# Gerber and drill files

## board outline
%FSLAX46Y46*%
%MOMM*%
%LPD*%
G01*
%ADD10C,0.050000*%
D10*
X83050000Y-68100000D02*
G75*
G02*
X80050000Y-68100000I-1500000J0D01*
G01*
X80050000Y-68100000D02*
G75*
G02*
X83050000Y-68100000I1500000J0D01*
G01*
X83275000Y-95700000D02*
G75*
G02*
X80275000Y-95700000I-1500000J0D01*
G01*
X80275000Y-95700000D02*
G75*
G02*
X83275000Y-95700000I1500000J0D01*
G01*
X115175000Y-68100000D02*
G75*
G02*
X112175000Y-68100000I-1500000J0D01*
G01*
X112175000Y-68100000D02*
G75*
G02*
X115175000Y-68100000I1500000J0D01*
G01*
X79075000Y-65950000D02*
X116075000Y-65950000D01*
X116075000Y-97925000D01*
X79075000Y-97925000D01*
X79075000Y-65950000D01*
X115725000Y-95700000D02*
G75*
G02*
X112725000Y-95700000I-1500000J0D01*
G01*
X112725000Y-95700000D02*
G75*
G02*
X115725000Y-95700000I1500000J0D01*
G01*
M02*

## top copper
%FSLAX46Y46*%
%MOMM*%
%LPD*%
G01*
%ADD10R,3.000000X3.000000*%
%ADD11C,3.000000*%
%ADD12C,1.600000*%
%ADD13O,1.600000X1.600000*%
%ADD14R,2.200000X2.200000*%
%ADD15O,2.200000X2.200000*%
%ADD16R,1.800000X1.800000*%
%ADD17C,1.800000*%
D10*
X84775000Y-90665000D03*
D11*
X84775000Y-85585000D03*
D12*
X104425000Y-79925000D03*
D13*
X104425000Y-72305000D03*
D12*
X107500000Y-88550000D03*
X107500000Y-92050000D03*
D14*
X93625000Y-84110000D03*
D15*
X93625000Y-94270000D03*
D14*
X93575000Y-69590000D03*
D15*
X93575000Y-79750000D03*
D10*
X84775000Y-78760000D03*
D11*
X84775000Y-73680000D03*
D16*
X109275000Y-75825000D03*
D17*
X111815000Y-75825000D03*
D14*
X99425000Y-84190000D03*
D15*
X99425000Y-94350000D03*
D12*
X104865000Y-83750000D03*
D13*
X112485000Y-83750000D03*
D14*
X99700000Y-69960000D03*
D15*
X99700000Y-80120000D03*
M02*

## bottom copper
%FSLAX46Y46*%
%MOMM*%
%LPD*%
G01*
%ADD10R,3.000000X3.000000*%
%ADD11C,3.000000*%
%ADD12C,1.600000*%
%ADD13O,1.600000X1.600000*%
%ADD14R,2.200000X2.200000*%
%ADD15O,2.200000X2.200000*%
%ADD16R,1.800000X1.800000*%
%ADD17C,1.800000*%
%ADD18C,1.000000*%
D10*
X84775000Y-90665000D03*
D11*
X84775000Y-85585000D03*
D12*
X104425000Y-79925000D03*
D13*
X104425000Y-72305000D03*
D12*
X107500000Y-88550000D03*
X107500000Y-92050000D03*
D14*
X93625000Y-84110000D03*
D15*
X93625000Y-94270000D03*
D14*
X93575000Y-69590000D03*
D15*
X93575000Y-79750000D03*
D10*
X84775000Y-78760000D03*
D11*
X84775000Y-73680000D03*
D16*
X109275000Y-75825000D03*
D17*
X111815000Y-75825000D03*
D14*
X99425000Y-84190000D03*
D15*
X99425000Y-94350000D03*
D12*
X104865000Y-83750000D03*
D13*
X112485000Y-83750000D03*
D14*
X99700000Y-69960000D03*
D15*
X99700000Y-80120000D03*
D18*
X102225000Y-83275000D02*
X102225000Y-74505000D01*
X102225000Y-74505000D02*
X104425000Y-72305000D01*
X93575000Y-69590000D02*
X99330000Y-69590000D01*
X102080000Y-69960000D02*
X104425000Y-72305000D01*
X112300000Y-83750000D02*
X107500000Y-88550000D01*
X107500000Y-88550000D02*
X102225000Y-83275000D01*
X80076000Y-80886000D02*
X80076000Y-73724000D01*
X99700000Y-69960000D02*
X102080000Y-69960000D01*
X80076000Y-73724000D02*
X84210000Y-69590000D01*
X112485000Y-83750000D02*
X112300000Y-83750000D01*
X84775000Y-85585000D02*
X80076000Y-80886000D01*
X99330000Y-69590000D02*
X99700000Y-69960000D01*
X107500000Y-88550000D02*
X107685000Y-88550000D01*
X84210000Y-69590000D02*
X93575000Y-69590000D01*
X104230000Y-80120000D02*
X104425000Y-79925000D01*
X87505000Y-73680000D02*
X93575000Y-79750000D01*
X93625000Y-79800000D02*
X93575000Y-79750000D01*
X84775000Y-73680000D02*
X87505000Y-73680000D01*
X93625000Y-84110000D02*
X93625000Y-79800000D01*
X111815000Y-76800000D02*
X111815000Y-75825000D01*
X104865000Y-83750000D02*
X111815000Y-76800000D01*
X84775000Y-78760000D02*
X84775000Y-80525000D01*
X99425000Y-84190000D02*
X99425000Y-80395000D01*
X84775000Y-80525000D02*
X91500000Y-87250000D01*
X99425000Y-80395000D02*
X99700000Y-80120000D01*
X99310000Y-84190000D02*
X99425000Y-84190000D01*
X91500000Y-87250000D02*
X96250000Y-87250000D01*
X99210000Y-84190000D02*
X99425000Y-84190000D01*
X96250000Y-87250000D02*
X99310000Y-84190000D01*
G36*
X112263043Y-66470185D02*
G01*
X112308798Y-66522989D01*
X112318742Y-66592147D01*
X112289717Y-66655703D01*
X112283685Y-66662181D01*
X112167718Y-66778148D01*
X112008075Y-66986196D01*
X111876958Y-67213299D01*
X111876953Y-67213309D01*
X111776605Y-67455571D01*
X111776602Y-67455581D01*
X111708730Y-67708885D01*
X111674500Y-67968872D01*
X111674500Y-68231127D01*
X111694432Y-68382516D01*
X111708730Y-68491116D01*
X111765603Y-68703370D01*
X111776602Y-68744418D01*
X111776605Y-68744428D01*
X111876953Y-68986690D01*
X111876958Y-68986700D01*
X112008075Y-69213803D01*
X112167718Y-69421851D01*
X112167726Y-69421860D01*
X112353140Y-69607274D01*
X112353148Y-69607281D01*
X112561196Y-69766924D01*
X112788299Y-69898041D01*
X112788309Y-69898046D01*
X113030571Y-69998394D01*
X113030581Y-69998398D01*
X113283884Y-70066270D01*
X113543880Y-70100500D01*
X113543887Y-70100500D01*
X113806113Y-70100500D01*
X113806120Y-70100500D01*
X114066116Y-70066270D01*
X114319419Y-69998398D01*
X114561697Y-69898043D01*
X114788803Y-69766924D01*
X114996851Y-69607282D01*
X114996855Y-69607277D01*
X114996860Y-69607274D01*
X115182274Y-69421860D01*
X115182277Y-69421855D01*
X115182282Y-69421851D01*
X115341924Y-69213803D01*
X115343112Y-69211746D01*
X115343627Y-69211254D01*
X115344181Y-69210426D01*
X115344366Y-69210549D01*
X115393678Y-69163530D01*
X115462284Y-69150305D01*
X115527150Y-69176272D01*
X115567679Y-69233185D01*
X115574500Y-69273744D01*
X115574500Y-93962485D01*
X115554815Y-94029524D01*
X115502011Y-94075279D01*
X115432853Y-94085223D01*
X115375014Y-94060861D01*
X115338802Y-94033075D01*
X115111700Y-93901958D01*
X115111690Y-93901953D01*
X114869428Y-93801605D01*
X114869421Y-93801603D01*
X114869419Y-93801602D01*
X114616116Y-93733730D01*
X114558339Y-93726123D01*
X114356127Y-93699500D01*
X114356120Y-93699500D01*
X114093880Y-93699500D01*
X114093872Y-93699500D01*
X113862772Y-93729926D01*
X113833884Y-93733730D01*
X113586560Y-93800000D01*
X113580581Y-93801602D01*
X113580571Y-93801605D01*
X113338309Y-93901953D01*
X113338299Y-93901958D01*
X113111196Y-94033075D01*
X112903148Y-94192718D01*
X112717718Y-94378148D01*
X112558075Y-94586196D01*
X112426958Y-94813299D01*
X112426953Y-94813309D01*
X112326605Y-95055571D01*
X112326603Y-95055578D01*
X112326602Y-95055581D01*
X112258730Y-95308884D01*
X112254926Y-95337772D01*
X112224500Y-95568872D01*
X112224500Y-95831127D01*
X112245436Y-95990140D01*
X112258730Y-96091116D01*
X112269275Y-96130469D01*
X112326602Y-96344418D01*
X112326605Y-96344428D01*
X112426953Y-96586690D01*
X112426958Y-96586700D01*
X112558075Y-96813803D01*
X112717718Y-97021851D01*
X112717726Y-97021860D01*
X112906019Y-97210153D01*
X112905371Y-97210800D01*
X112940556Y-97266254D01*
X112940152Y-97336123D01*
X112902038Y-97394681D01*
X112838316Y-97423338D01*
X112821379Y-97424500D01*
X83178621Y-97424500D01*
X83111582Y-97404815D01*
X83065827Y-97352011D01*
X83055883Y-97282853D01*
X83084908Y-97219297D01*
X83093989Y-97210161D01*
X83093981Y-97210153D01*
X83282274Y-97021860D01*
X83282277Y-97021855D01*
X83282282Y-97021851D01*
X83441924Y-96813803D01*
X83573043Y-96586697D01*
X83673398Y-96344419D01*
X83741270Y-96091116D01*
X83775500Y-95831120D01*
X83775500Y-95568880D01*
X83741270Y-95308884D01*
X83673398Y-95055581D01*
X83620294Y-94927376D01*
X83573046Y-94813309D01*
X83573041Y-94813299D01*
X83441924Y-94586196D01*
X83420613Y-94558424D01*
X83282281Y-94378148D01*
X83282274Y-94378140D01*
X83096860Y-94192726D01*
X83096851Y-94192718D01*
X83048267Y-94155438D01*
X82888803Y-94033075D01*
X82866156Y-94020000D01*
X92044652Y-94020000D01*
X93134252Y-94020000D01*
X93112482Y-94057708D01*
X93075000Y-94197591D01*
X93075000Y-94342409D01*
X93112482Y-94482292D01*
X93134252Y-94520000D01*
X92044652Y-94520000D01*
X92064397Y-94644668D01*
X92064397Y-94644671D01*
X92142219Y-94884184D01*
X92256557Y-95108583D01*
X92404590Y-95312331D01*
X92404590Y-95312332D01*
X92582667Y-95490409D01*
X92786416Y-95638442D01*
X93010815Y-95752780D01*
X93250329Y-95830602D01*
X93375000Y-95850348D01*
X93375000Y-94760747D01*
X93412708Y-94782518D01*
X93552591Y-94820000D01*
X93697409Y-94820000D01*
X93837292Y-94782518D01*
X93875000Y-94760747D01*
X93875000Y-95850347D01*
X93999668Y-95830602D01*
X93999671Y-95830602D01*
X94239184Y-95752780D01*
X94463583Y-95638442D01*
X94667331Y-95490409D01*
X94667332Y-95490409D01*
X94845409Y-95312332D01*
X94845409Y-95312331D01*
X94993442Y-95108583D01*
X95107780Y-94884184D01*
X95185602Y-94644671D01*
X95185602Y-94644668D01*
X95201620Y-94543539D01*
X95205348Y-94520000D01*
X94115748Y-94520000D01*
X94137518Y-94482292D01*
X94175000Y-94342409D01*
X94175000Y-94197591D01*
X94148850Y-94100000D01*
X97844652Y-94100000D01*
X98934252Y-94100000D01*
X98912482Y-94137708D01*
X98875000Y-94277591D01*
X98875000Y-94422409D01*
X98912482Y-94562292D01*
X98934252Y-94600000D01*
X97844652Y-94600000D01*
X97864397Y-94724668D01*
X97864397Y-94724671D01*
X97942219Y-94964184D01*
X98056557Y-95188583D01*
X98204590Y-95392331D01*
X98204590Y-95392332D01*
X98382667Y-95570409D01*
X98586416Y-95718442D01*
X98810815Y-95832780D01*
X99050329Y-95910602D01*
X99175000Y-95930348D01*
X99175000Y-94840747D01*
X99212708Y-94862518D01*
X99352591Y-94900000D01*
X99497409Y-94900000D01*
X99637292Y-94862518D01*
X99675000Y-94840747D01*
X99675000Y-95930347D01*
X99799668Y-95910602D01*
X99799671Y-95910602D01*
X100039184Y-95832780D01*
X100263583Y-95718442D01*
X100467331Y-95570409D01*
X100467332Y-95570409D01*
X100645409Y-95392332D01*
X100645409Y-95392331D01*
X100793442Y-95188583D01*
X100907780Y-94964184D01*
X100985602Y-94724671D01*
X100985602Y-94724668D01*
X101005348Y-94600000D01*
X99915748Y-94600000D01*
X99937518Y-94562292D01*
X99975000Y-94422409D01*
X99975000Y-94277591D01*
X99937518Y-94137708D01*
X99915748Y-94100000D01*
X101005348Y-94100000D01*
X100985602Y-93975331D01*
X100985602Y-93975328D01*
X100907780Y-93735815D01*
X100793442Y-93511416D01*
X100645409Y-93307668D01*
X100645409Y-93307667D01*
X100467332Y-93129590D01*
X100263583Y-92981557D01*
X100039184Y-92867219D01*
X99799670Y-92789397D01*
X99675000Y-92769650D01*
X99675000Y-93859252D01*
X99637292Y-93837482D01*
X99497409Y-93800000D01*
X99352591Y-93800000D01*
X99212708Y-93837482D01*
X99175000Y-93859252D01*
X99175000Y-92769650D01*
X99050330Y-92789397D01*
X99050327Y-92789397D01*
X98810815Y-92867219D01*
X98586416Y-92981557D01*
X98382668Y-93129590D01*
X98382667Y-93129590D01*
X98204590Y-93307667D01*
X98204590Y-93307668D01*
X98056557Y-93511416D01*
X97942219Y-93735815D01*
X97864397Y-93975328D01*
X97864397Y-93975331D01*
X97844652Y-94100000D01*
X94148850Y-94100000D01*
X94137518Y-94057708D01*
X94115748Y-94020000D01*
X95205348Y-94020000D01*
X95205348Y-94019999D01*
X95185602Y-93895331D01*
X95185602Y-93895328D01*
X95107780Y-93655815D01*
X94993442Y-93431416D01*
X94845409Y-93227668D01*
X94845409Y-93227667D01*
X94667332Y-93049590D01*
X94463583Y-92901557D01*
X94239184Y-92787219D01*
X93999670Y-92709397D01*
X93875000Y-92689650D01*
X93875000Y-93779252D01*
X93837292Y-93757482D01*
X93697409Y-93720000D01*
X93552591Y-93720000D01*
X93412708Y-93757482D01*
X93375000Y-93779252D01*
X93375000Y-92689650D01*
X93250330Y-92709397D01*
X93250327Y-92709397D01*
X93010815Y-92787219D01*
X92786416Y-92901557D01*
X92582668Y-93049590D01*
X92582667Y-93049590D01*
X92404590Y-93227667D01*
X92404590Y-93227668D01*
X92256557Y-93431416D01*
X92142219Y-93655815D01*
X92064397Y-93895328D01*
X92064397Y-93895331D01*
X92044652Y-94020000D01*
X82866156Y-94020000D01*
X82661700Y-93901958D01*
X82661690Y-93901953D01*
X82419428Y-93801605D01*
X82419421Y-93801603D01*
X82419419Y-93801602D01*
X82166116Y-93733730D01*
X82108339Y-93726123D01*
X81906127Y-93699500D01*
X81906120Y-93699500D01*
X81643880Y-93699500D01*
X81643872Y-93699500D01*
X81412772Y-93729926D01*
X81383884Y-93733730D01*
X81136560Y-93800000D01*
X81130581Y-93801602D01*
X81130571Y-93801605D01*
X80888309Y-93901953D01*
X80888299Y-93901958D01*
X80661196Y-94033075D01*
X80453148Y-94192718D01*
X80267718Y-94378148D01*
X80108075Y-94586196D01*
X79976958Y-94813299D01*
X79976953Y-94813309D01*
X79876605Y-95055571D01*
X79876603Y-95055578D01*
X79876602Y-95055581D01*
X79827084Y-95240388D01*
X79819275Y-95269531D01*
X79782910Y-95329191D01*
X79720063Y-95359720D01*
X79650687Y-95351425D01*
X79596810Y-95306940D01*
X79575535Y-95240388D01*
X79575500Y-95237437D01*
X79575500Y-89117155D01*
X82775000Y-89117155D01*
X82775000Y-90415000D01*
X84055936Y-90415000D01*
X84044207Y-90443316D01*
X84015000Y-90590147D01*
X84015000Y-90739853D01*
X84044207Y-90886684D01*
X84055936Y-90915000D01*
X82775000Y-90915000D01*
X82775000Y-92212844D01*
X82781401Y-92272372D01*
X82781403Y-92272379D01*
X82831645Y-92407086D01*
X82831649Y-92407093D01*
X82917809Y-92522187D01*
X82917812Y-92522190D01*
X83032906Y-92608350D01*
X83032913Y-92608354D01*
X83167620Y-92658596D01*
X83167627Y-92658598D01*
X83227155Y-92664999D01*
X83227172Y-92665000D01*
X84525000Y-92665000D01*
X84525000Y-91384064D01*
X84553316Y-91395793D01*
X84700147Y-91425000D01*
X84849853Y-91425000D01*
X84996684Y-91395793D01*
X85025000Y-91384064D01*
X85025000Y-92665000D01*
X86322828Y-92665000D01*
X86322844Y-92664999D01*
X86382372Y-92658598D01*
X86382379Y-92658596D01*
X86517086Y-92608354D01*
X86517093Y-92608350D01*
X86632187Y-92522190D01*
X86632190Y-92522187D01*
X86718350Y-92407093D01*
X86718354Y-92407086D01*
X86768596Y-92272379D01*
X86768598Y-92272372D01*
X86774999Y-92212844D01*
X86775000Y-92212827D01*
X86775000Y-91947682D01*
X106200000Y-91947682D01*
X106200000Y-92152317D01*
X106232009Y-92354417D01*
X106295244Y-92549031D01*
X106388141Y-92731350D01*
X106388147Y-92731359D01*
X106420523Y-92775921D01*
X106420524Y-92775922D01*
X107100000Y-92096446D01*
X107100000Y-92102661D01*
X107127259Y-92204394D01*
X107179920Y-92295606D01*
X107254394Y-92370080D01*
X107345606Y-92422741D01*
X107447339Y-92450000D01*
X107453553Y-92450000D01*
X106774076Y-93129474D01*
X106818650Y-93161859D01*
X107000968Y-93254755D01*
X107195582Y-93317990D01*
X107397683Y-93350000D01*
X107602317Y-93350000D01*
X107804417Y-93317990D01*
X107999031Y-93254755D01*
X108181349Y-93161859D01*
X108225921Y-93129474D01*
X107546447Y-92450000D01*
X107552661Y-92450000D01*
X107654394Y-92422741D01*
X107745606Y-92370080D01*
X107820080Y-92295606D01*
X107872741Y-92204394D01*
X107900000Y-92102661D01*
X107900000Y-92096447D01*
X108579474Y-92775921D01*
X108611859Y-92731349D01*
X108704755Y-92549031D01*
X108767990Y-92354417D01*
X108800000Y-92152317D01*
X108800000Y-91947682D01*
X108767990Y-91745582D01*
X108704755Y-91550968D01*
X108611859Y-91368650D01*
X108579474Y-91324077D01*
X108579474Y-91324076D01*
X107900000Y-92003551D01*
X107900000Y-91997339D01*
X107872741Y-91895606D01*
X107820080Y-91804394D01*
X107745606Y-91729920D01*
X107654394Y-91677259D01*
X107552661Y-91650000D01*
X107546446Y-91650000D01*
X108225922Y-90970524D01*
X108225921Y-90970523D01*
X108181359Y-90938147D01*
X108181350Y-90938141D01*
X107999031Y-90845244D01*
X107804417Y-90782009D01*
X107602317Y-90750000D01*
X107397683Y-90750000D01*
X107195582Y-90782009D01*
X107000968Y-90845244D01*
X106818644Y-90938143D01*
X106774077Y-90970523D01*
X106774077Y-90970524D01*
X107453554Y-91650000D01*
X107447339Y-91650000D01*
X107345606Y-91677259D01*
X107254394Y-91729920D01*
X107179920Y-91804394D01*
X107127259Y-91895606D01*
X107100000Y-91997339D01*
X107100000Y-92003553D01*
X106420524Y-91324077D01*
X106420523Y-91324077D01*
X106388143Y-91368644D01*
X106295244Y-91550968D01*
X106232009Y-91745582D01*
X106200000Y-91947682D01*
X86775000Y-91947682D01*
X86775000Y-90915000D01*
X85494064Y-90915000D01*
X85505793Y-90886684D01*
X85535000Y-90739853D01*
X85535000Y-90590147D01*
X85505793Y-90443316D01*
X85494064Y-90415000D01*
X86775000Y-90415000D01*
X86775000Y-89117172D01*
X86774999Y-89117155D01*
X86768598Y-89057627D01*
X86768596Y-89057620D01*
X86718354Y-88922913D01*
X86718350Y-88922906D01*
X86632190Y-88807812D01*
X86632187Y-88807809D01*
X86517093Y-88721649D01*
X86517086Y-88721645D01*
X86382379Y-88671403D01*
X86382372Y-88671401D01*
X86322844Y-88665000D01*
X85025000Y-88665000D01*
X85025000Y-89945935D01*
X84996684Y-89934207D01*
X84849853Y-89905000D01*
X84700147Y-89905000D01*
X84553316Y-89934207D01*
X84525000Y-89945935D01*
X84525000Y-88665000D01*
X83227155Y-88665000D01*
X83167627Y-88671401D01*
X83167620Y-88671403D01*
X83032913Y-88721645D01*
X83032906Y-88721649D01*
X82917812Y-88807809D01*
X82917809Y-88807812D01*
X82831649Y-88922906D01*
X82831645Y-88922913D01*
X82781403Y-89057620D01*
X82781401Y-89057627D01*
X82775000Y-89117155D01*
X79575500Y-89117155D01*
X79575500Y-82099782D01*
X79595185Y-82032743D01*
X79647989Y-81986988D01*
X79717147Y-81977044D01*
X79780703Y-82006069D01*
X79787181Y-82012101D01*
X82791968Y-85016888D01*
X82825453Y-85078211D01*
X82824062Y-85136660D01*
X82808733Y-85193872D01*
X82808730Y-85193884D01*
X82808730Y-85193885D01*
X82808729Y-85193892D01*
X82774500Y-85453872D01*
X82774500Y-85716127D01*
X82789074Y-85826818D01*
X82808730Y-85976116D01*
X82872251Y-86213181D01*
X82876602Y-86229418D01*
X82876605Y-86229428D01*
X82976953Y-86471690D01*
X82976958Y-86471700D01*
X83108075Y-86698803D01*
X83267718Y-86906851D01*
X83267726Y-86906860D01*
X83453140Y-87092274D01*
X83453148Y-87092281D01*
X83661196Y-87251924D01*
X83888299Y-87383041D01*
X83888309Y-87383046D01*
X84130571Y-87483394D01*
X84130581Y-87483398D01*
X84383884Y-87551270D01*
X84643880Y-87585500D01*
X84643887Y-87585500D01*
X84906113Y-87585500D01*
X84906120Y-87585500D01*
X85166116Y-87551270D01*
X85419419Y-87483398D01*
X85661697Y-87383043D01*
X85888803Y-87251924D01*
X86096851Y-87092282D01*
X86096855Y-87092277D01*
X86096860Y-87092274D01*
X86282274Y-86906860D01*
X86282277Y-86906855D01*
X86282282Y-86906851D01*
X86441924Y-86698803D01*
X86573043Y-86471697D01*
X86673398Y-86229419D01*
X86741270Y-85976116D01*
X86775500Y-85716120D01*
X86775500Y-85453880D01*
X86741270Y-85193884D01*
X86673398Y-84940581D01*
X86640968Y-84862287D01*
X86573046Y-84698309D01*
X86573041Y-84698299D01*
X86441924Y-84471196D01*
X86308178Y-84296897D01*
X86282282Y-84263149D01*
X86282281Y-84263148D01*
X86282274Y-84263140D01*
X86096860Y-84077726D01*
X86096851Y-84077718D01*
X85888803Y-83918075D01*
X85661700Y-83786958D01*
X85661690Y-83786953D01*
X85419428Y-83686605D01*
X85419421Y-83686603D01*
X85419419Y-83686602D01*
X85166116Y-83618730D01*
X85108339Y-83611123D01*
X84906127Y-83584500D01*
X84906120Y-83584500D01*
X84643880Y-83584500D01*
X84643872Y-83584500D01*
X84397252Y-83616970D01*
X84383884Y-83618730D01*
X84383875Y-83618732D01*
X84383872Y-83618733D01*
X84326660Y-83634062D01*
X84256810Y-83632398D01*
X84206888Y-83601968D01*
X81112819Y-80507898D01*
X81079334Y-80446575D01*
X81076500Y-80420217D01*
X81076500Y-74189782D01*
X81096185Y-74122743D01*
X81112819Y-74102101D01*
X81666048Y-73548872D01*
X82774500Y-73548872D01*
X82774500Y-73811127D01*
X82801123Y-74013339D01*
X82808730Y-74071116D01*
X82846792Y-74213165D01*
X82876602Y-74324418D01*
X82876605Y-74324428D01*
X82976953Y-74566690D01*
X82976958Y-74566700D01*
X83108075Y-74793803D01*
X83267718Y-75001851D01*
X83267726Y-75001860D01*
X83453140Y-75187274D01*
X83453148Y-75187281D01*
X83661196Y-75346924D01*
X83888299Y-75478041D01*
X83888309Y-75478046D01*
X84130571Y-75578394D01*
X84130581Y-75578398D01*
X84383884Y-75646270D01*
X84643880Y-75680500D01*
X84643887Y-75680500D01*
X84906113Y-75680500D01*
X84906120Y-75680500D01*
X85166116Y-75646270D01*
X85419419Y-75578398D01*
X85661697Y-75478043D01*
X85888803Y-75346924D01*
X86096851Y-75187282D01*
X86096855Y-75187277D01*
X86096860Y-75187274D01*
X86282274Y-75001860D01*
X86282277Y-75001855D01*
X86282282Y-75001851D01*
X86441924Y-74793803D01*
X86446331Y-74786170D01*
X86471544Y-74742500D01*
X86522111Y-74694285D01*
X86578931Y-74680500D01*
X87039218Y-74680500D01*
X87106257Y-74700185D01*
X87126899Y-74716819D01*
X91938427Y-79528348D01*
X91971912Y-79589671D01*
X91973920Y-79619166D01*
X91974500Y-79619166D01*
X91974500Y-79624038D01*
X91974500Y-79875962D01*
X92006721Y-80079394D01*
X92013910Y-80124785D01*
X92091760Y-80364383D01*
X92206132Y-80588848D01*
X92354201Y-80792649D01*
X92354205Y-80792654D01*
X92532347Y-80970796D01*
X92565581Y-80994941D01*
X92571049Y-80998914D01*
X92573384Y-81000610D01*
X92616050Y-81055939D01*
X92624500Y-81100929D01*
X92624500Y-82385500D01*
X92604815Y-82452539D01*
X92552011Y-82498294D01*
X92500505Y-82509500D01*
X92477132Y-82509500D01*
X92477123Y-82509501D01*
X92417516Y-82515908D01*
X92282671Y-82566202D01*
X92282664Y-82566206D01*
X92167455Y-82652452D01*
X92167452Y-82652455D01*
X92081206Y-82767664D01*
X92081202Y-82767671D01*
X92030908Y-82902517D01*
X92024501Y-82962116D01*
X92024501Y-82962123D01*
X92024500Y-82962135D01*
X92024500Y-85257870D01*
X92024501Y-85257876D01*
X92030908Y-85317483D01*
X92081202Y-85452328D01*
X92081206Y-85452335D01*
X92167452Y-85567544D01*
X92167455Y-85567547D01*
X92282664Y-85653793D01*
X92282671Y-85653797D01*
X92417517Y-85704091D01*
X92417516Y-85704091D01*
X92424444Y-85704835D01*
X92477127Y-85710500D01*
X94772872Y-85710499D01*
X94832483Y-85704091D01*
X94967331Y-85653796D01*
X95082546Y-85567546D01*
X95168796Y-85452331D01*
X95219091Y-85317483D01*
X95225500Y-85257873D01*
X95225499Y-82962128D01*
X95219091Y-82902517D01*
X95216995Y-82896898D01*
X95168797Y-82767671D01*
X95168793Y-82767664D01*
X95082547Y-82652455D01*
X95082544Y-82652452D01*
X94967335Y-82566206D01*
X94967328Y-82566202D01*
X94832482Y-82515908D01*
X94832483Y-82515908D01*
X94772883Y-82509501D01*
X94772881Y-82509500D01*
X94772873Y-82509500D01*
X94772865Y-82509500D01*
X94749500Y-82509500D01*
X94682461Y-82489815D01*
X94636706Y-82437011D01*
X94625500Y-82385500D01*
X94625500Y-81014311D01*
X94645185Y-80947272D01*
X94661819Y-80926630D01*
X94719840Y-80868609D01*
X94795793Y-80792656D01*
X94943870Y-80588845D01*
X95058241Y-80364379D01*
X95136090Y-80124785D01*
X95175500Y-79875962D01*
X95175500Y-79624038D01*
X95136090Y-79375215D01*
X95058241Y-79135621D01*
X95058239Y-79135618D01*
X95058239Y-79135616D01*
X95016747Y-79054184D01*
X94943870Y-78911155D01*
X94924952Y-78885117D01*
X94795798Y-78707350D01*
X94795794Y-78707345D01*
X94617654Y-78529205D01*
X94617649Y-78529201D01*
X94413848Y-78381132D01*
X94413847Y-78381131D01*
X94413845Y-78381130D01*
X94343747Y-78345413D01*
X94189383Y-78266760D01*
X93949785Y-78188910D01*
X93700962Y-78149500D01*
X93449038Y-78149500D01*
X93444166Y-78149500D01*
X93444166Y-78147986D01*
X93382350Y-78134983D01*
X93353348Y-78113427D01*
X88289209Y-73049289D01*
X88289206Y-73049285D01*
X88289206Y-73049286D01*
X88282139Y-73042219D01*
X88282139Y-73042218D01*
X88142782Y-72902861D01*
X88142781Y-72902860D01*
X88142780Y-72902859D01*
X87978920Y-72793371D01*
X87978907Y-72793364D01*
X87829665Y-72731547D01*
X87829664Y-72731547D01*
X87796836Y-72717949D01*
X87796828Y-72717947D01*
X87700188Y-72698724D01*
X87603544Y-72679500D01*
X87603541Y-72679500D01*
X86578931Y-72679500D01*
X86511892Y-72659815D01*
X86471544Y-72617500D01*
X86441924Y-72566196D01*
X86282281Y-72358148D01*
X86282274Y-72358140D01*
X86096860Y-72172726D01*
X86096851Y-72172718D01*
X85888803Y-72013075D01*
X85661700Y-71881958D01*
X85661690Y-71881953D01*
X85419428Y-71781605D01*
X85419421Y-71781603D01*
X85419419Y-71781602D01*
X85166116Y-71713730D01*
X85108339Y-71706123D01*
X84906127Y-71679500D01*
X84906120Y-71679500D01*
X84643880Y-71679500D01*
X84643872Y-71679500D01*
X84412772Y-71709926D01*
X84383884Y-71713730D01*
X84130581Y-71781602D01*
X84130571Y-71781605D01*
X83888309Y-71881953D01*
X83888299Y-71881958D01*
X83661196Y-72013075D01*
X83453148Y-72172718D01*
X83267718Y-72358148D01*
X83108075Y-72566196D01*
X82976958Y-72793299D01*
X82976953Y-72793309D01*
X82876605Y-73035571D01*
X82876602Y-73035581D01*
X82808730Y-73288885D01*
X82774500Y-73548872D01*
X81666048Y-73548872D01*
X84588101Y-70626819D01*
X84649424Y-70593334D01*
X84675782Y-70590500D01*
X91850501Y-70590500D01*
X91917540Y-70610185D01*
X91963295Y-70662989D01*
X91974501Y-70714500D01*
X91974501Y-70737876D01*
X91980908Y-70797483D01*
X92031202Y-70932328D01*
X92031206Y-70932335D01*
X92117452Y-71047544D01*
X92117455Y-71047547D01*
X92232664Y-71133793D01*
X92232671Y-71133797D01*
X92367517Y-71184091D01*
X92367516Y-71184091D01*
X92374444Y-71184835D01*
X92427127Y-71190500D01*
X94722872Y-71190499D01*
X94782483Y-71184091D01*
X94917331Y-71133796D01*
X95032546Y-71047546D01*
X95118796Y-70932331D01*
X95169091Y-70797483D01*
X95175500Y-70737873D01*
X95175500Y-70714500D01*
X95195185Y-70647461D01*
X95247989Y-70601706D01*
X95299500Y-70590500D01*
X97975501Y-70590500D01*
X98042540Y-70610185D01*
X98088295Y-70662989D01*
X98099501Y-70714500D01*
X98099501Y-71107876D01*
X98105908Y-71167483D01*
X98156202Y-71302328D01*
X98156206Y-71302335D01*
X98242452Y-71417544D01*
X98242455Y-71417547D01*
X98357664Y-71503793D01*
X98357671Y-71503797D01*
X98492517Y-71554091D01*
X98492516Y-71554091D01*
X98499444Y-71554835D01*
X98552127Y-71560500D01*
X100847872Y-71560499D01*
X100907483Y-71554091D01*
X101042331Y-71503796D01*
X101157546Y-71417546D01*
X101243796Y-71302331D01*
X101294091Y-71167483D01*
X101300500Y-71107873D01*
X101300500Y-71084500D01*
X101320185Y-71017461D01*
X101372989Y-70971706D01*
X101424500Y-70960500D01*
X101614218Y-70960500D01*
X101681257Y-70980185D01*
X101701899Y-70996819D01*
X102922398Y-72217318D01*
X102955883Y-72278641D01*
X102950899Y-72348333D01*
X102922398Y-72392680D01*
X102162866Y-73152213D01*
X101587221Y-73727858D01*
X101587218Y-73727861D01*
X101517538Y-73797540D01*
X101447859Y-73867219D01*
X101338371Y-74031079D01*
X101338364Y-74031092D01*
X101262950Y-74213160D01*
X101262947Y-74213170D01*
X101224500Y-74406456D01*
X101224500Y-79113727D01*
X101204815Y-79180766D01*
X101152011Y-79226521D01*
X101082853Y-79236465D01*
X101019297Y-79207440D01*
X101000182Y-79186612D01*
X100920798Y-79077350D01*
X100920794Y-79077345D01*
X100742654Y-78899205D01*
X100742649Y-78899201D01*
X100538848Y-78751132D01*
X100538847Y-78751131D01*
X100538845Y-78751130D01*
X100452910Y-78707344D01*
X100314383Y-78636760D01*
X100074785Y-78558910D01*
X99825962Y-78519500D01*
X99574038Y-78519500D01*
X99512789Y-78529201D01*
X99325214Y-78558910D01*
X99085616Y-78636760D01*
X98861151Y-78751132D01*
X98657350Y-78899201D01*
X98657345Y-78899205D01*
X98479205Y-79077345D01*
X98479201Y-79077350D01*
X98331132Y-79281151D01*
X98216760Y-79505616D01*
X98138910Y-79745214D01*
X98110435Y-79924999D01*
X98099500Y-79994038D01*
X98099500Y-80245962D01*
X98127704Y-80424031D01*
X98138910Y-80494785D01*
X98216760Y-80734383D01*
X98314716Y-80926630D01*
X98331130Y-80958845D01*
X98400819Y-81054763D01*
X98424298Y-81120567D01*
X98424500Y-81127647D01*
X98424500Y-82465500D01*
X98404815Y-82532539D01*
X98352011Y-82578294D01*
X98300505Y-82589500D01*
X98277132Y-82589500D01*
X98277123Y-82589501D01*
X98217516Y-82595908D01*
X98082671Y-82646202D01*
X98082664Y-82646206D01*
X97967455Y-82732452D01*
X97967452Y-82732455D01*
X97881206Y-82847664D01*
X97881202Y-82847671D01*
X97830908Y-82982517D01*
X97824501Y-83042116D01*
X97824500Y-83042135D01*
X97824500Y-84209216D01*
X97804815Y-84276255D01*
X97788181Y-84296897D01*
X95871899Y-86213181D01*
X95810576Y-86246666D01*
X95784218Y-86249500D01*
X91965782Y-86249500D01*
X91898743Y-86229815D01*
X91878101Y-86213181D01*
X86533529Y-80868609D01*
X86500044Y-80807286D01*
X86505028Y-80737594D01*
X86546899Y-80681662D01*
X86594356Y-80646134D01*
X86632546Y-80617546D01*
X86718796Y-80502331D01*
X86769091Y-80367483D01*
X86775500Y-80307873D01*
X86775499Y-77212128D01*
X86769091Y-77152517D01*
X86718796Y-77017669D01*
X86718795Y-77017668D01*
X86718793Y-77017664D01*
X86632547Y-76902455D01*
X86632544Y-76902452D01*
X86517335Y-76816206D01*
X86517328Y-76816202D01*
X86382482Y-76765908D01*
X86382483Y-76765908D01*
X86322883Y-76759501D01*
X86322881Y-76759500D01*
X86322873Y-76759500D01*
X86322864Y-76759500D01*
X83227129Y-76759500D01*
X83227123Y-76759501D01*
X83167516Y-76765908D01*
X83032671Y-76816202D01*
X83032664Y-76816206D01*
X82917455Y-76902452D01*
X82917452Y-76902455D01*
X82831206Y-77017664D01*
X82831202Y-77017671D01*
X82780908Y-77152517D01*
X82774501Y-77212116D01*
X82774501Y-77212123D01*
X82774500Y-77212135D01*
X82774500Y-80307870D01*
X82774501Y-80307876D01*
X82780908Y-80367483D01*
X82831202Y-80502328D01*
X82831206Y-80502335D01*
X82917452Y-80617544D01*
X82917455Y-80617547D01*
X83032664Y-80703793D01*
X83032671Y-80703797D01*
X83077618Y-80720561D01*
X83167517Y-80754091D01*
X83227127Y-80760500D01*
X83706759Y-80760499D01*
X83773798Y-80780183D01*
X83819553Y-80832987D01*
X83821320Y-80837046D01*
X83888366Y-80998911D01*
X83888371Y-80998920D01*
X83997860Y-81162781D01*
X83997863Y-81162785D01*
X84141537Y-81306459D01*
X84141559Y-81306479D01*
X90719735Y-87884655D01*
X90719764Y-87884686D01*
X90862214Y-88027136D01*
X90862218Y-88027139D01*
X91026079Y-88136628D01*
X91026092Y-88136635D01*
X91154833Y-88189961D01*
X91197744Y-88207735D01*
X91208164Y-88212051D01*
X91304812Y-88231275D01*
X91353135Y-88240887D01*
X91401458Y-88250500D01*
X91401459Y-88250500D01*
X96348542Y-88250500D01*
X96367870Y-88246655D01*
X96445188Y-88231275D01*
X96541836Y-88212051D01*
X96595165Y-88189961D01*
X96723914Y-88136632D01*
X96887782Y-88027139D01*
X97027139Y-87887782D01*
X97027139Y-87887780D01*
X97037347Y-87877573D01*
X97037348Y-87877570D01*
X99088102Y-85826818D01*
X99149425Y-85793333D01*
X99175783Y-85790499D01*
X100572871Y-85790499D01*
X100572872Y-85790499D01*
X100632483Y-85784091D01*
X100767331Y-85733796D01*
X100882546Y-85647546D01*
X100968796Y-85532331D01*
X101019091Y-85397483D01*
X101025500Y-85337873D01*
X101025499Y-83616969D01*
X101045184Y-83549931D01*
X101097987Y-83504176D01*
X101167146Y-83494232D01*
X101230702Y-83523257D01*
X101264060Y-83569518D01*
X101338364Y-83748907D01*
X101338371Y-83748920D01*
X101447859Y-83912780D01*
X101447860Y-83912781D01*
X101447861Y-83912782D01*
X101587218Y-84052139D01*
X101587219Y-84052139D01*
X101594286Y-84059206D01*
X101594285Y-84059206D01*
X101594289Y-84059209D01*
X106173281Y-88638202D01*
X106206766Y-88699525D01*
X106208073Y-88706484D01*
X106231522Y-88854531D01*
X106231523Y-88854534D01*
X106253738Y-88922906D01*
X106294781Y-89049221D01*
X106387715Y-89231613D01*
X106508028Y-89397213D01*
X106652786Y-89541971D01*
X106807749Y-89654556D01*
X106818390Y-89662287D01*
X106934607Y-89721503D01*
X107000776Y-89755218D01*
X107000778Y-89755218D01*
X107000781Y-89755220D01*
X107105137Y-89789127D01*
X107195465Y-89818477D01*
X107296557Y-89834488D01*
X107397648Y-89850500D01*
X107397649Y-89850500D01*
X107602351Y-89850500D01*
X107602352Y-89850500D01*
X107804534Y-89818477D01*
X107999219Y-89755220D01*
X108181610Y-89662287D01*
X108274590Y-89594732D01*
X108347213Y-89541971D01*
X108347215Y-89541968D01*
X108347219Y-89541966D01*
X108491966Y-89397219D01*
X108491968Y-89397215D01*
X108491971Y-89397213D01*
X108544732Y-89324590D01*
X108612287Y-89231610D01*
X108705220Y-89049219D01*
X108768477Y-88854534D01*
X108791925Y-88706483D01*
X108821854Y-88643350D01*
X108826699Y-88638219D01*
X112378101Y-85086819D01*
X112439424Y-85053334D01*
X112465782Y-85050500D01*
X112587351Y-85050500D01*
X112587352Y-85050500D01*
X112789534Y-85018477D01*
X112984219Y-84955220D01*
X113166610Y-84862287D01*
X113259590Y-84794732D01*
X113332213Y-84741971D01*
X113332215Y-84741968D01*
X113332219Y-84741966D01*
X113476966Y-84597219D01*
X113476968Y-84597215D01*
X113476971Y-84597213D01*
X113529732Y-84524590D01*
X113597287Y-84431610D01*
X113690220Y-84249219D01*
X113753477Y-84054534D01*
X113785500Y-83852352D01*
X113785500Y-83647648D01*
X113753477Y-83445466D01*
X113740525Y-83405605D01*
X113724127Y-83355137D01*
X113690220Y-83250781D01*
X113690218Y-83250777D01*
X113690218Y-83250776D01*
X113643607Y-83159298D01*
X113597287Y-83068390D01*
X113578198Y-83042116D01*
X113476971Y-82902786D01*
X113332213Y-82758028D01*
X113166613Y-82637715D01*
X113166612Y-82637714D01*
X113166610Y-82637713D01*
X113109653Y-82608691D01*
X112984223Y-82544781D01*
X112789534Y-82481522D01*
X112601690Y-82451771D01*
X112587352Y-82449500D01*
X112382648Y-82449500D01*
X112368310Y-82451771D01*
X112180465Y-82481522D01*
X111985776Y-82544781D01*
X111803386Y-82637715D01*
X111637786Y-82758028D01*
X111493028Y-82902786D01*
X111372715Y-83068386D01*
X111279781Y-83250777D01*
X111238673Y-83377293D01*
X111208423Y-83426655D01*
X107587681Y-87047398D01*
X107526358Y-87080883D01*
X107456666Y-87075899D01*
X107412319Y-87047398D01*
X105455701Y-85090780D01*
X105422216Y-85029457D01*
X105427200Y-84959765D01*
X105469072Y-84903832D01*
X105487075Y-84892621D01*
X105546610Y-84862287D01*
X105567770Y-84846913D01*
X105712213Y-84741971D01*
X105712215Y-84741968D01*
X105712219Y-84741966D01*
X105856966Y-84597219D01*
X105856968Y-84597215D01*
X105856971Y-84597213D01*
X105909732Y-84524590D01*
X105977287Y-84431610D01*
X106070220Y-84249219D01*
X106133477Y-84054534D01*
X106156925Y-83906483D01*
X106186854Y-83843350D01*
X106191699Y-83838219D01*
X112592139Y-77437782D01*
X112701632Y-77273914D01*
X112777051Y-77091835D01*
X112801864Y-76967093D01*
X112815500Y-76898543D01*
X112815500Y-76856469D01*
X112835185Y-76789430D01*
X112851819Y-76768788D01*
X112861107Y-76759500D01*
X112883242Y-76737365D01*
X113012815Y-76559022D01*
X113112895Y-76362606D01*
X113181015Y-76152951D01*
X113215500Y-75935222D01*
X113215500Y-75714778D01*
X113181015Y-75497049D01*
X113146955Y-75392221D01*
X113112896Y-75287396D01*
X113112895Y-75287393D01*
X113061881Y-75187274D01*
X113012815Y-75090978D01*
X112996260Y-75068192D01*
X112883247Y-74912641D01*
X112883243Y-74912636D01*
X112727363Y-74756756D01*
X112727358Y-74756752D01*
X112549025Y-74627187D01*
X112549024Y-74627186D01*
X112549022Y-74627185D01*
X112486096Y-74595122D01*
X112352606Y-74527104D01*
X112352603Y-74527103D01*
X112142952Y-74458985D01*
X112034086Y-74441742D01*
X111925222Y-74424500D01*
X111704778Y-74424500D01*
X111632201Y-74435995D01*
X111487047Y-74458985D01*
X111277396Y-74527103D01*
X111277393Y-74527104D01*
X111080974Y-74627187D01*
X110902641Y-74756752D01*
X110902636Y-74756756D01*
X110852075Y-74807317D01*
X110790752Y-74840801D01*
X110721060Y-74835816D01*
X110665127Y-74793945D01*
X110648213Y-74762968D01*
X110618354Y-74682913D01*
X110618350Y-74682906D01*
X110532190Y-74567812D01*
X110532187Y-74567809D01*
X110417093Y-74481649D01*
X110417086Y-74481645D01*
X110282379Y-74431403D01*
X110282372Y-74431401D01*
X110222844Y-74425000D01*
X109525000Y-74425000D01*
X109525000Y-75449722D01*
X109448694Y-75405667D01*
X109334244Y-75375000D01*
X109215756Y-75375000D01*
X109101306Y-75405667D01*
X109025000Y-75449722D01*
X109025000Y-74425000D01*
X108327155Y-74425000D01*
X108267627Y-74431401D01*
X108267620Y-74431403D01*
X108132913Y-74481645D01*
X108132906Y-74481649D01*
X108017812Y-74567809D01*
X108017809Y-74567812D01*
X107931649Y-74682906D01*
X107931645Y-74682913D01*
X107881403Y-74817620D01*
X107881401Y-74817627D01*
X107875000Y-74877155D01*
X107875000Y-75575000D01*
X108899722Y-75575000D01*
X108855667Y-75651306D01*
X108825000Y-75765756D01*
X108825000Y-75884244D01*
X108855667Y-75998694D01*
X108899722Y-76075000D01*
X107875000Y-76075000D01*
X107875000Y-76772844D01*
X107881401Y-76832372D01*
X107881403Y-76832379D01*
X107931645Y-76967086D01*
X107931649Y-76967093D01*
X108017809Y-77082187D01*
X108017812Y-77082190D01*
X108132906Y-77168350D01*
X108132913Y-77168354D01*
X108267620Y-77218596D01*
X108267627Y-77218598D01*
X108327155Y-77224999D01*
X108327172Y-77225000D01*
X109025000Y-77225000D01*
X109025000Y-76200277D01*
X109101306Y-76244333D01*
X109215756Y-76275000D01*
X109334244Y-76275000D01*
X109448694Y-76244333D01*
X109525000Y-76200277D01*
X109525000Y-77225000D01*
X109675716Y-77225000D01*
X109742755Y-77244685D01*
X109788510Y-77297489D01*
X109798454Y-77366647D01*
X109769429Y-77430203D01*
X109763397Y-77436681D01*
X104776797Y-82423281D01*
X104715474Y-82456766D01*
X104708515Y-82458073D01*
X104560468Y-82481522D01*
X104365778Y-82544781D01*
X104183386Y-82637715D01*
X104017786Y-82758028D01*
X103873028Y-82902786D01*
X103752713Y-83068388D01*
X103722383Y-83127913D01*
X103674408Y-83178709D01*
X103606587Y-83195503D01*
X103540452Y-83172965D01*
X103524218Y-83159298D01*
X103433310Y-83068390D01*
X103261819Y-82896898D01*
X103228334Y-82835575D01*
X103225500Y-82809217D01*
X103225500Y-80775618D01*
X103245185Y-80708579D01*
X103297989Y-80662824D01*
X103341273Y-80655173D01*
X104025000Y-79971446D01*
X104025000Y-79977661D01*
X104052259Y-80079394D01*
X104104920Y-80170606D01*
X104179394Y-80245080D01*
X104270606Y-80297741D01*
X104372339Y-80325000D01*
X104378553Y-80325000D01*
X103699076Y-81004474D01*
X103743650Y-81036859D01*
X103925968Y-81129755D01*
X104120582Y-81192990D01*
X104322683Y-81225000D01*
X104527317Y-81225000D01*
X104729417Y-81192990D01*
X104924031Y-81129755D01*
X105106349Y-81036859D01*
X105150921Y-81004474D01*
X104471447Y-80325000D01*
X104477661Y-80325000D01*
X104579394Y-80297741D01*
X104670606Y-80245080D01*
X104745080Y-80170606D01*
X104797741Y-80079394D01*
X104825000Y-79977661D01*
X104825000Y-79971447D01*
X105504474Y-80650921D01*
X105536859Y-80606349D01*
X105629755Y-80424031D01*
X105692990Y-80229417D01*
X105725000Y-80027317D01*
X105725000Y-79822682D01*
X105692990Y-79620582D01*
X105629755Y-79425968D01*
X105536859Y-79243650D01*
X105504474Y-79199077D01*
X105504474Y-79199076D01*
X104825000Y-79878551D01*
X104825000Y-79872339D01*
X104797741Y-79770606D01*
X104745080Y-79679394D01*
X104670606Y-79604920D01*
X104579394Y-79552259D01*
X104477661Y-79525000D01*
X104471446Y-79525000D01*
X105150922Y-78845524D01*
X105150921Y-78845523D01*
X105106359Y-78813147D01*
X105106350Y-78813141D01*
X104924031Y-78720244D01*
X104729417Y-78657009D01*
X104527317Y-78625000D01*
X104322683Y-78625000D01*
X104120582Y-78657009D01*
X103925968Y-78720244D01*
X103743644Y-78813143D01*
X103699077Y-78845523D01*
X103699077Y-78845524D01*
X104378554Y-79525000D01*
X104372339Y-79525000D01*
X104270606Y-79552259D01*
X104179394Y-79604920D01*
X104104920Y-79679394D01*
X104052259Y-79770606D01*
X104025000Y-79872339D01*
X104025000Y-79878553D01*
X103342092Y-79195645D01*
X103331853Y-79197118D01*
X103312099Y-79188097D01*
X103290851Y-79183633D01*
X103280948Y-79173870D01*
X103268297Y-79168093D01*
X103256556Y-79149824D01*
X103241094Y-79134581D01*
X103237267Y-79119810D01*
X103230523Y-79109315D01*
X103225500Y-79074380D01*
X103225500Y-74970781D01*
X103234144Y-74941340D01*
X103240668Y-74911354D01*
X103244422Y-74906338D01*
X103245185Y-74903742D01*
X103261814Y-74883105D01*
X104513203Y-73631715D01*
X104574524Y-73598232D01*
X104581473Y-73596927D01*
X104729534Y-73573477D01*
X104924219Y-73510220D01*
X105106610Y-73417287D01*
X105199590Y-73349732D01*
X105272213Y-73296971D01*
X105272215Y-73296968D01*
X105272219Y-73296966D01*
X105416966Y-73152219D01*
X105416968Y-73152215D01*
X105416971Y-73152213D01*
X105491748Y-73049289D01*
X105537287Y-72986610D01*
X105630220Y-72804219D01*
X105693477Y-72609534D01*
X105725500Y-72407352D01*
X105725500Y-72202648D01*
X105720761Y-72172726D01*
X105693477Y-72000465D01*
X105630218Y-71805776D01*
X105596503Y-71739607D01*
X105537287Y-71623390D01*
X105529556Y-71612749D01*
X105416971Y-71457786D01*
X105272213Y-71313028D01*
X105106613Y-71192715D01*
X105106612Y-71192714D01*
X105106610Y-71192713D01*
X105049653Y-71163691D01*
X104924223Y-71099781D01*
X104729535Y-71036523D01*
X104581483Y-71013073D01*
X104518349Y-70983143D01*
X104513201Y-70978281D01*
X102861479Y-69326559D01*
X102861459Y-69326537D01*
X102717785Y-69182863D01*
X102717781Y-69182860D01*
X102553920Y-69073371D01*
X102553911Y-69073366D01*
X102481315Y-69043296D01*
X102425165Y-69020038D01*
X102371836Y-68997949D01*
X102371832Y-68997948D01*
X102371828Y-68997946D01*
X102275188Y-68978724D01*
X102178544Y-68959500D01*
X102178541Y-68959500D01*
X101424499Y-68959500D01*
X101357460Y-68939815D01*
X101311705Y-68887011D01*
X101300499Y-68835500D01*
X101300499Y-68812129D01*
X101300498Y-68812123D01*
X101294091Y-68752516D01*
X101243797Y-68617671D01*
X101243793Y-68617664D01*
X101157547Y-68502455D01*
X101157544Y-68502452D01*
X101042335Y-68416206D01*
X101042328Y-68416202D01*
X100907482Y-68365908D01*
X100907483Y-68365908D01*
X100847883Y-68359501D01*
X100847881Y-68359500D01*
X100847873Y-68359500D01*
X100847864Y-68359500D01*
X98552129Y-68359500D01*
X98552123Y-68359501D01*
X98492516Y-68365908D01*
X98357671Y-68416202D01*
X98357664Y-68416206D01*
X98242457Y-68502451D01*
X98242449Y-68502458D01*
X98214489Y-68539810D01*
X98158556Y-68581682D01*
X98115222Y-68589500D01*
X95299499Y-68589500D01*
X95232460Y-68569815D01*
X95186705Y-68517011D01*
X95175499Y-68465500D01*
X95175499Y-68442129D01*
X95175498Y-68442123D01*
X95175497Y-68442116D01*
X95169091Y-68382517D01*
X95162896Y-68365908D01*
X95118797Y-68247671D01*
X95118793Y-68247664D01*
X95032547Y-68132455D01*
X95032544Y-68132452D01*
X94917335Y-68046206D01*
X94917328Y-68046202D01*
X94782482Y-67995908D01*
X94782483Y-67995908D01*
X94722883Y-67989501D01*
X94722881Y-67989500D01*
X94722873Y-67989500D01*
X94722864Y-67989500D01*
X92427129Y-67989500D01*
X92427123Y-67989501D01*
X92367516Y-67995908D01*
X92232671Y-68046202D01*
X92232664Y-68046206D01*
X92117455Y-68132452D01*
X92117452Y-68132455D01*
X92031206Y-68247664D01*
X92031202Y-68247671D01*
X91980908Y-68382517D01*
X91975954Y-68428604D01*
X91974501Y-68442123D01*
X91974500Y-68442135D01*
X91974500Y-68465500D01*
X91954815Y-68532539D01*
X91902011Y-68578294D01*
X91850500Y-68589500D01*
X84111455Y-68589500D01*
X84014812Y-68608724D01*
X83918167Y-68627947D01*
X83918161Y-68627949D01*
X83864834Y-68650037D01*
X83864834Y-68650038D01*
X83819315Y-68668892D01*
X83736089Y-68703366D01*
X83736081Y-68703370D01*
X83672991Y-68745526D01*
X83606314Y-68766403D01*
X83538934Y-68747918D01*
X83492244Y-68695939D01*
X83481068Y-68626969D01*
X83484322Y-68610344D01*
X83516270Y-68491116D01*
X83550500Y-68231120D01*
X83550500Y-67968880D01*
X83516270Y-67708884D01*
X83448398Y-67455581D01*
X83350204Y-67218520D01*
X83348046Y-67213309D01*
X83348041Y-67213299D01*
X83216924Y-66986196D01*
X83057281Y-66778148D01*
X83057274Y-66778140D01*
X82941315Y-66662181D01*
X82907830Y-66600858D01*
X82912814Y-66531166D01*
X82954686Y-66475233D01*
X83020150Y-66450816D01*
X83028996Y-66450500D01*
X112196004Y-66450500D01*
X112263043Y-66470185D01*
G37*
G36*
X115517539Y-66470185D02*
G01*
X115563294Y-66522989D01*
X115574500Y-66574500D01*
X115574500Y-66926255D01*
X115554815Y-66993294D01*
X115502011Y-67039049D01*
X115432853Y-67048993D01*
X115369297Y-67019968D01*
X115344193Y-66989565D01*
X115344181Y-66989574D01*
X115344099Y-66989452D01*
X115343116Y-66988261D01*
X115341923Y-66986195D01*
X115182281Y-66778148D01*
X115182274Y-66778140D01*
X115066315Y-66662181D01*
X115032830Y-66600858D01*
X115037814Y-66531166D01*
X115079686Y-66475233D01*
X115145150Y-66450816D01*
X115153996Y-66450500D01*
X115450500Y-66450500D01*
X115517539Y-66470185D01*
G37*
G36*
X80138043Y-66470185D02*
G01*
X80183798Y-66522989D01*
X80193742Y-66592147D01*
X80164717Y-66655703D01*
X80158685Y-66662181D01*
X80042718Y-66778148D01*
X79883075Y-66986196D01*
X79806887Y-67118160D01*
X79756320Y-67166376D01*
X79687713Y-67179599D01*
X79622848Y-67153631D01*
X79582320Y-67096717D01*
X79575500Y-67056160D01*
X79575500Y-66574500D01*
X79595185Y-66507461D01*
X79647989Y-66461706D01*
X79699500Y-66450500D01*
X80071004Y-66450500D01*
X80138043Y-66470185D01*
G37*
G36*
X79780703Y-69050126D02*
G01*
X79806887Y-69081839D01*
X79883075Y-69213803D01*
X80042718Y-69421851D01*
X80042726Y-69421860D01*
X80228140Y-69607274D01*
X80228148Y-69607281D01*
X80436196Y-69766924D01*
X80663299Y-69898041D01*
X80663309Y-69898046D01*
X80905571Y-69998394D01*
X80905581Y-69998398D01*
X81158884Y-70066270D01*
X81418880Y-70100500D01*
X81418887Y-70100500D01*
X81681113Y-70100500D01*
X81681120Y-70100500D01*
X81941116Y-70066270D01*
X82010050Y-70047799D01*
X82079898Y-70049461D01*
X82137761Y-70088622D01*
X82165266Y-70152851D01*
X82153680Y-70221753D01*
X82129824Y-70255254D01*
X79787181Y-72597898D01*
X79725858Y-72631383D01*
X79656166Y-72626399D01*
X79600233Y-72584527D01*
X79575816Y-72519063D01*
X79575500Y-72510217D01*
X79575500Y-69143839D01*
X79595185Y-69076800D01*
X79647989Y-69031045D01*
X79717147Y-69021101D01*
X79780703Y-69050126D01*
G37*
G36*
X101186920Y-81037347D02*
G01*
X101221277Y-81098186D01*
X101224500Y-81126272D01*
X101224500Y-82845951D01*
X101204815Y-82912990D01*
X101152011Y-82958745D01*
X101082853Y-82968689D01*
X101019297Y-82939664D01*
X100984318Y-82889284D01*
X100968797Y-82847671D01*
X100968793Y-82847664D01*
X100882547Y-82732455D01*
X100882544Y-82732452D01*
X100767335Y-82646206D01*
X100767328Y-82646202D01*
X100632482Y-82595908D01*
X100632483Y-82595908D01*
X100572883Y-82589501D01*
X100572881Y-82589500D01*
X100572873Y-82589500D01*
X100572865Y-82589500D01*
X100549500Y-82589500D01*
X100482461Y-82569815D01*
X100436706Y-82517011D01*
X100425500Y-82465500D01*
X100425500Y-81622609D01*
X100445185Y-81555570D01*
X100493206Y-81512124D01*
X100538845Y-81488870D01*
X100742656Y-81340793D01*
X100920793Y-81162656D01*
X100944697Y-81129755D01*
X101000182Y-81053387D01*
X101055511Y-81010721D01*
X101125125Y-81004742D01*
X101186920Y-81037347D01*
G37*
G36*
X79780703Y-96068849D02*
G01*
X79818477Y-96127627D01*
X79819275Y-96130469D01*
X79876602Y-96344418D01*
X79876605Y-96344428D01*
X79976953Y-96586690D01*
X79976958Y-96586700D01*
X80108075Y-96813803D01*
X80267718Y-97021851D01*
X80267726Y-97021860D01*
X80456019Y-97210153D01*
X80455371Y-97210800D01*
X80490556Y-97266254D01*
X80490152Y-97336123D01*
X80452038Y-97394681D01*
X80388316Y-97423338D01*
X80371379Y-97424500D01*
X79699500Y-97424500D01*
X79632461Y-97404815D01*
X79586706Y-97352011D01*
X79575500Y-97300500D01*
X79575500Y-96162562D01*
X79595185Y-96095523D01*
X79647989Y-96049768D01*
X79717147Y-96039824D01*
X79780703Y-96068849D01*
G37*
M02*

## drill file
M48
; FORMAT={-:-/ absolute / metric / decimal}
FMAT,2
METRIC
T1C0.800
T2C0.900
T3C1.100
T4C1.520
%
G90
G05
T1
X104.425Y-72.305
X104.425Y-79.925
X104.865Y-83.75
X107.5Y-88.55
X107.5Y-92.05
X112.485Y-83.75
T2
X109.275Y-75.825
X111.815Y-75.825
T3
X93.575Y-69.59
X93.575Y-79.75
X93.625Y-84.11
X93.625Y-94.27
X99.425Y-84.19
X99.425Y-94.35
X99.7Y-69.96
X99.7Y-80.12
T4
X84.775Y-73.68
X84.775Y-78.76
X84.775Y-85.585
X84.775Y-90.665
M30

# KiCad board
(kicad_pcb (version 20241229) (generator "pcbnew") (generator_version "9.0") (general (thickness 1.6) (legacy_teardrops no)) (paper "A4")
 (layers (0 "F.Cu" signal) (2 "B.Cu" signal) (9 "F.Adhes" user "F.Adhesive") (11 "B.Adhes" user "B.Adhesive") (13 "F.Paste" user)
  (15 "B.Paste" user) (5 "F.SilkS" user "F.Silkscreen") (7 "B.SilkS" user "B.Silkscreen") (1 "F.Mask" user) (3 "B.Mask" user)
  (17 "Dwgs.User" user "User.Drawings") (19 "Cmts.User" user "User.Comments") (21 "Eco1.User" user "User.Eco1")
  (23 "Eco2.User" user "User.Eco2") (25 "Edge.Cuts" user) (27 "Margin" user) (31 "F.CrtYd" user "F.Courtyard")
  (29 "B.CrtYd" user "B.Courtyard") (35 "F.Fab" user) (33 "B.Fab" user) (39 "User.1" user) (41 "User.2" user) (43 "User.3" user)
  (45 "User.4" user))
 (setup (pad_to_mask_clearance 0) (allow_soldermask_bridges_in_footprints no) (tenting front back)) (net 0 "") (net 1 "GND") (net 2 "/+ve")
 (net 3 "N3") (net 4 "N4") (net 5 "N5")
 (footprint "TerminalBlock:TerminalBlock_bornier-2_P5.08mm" (layer "F.Cu") (at 84.775 90.665 90)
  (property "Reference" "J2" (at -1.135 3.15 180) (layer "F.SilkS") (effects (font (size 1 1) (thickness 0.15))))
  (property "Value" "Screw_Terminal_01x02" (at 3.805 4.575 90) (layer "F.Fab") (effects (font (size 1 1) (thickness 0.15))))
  (pad "1" thru_hole rect (at 0 0 90) (size 3 3) (drill 1.52) (layers "*.Cu" "*.Mask") (remove_unused_layers no) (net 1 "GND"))
  (pad "2" thru_hole circle (at 5.08 0 90) (size 3 3) (drill 1.52) (layers "*.Cu" "*.Mask") (remove_unused_layers no) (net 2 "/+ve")))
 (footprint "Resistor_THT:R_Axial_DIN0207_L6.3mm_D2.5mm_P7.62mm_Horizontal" (layer "F.Cu") (at 104.425 79.925 90)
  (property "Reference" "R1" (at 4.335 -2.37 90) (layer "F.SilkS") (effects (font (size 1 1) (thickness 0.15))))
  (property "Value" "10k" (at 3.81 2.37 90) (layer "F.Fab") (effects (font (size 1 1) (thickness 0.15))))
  (pad "1" thru_hole circle (at 0 0 90) (size 1.6 1.6) (drill 0.8) (layers "*.Cu" "*.Mask") (remove_unused_layers no) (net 1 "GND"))
  (pad "2" thru_hole oval (at 7.62 0 90) (size 1.6 1.6) (drill 0.8) (layers "*.Cu" "*.Mask") (remove_unused_layers no) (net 2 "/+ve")))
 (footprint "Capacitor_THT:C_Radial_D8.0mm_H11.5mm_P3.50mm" (layer "F.Cu") (at 107.5 88.55 -90)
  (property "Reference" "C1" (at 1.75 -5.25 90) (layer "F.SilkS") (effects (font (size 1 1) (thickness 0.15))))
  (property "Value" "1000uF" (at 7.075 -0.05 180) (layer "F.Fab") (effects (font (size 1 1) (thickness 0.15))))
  (pad "1" thru_hole circle (at 0 0 270) (size 1.6 1.6) (drill 0.8) (layers "*.Cu" "*.Mask") (remove_unused_layers no) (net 2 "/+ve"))
  (pad "2" thru_hole circle (at 3.5 0 270) (size 1.6 1.6) (drill 0.8) (layers "*.Cu" "*.Mask") (remove_unused_layers no) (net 1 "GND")))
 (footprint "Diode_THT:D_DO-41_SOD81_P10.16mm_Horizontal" (layer "F.Cu") (at 93.625 84.11 -90)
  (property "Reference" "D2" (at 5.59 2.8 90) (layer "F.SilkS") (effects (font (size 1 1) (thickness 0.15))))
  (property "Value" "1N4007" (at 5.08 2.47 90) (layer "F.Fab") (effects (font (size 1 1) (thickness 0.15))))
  (pad "1" thru_hole rect (at 0 0 270) (size 2.2 2.2) (drill 1.1) (layers "*.Cu" "*.Mask") (remove_unused_layers no) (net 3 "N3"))
  (pad "2" thru_hole oval (at 10.16 0 270) (size 2.2 2.2) (drill 1.1) (layers "*.Cu" "*.Mask") (remove_unused_layers no) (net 1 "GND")))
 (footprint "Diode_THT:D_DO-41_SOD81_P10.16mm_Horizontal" (layer "F.Cu") (at 93.575 69.59 -90)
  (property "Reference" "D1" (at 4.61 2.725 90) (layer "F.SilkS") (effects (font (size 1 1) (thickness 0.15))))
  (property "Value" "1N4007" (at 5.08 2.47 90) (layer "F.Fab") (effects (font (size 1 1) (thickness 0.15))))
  (pad "1" thru_hole rect (at 0 0 270) (size 2.2 2.2) (drill 1.1) (layers "*.Cu" "*.Mask") (remove_unused_layers no) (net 2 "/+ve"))
  (pad "2" thru_hole oval (at 10.16 0 270) (size 2.2 2.2) (drill 1.1) (layers "*.Cu" "*.Mask") (remove_unused_layers no) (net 3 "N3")))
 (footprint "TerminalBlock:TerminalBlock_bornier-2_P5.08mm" (layer "F.Cu") (at 84.775 78.76 90)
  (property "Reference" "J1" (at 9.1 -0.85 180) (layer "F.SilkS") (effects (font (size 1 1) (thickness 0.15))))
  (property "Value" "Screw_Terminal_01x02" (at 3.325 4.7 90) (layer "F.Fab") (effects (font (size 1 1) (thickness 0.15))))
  (pad "1" thru_hole rect (at 0 0 90) (size 3 3) (drill 1.52) (layers "*.Cu" "*.Mask") (remove_unused_layers no) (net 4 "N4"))
  (pad "2" thru_hole circle (at 5.08 0 90) (size 3 3) (drill 1.52) (layers "*.Cu" "*.Mask") (remove_unused_layers no) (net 3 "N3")))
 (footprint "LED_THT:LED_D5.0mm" (layer "F.Cu") (at 109.275 75.825)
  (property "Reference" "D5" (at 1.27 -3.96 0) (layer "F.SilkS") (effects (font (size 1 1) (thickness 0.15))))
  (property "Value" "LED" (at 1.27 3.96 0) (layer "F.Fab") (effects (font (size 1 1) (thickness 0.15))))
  (pad "1" thru_hole rect (at 0 0) (size 1.8 1.8) (drill 0.9) (layers "*.Cu" "*.Mask") (remove_unused_layers no) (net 1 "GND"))
  (pad "2" thru_hole circle (at 2.54 0) (size 1.8 1.8) (drill 0.9) (layers "*.Cu" "*.Mask") (remove_unused_layers no) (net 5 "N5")))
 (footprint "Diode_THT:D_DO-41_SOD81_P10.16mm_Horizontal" (layer "F.Cu") (at 99.425 84.19 -90)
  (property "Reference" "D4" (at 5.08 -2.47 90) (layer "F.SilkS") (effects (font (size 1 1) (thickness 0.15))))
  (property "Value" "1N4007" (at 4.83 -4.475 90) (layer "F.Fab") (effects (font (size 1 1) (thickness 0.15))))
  (pad "1" thru_hole rect (at 0 0 270) (size 2.2 2.2) (drill 1.1) (layers "*.Cu" "*.Mask") (remove_unused_layers no) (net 4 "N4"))
  (pad "2" thru_hole oval (at 10.16 0 270) (size 2.2 2.2) (drill 1.1) (layers "*.Cu" "*.Mask") (remove_unused_layers no) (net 1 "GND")))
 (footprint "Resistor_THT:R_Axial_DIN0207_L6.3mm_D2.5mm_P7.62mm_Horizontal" (layer "F.Cu") (at 104.865 83.75)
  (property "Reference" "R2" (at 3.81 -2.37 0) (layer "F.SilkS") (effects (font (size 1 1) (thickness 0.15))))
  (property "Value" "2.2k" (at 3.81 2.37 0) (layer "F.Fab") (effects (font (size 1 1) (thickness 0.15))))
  (pad "1" thru_hole circle (at 0 0) (size 1.6 1.6) (drill 0.8) (layers "*.Cu" "*.Mask") (remove_unused_layers no) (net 5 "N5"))
  (pad "2" thru_hole oval (at 7.62 0) (size 1.6 1.6) (drill 0.8) (layers "*.Cu" "*.Mask") (remove_unused_layers no) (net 2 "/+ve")))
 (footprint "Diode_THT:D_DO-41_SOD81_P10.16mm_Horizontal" (layer "F.Cu") (at 99.7 69.96 -90)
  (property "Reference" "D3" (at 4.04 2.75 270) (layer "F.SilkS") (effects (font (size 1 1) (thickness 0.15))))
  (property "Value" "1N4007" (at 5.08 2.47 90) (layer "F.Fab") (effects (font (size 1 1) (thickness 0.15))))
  (pad "1" thru_hole rect (at 0 0 270) (size 2.2 2.2) (drill 1.1) (layers "*.Cu" "*.Mask") (remove_unused_layers no) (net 2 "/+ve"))
  (pad "2" thru_hole oval (at 10.16 0 270) (size 2.2 2.2) (drill 1.1) (layers "*.Cu" "*.Mask") (remove_unused_layers no) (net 4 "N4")))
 (gr_circle (center 81.55 68.1) (end 81.55 66.6) (stroke (width 0.05) (type default)) (fill no) (layer "Edge.Cuts"))
 (gr_circle (center 81.775 95.7) (end 81.775 94.2) (stroke (width 0.05) (type default)) (fill no) (layer "Edge.Cuts"))
 (gr_circle (center 113.675 68.1) (end 113.675 66.6) (stroke (width 0.05) (type default)) (fill no) (layer "Edge.Cuts"))
 (gr_rect (start 79.075 65.95) (end 116.075 97.925) (stroke (width 0.05) (type default)) (fill no) (layer "Edge.Cuts"))
 (gr_circle (center 114.225 95.7) (end 114.225 94.2) (stroke (width 0.05) (type default)) (fill no) (layer "Edge.Cuts"))
 (segment (start 102.225 83.275) (end 102.225 74.505) (width 1) (layer "B.Cu") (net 2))
 (segment (start 102.225 74.505) (end 104.425 72.305) (width 1) (layer "B.Cu") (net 2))
 (segment (start 93.575 69.59) (end 99.33 69.59) (width 1) (layer "B.Cu") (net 2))
 (segment (start 102.08 69.96) (end 104.425 72.305) (width 1) (layer "B.Cu") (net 2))
 (segment (start 112.3 83.75) (end 107.5 88.55) (width 1) (layer "B.Cu") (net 2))
 (segment (start 107.5 88.55) (end 102.225 83.275) (width 1) (layer "B.Cu") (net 2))
 (segment (start 80.076 80.886) (end 80.076 73.724) (width 1) (layer "B.Cu") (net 2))
 (segment (start 99.7 69.96) (end 102.08 69.96) (width 1) (layer "B.Cu") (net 2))
 (segment (start 80.076 73.724) (end 84.21 69.59) (width 1) (layer "B.Cu") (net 2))
 (segment (start 112.485 83.75) (end 112.3 83.75) (width 1) (layer "B.Cu") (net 2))
 (segment (start 84.775 85.585) (end 80.076 80.886) (width 1) (layer "B.Cu") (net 2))
 (segment (start 99.33 69.59) (end 99.7 69.96) (width 1) (layer "B.Cu") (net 2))
 (segment (start 107.5 88.55) (end 107.685 88.55) (width 1) (layer "B.Cu") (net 2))
 (segment (start 84.21 69.59) (end 93.575 69.59) (width 1) (layer "B.Cu") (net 2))
 (segment (start 104.23 80.12) (end 104.425 79.925) (width 1) (layer "B.Cu") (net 1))
 (segment (start 87.505 73.68) (end 93.575 79.75) (width 1) (layer "B.Cu") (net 3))
 (segment (start 93.625 79.8) (end 93.575 79.75) (width 1) (layer "B.Cu") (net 3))
 (segment (start 84.775 73.68) (end 87.505 73.68) (width 1) (layer "B.Cu") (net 3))
 (segment (start 93.625 84.11) (end 93.625 79.8) (width 1) (layer "B.Cu") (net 3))
 (segment (start 111.815 76.8) (end 111.815 75.825) (width 1) (layer "B.Cu") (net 5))
 (segment (start 104.865 83.75) (end 111.815 76.8) (width 1) (layer "B.Cu") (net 5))
 (segment (start 84.775 78.76) (end 84.775 80.525) (width 1) (layer "B.Cu") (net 4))
 (segment (start 99.425 84.19) (end 99.425 80.395) (width 1) (layer "B.Cu") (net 4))
 (segment (start 84.775 80.525) (end 91.5 87.25) (width 1) (layer "B.Cu") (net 4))
 (segment (start 99.425 80.395) (end 99.7 80.12) (width 1) (layer "B.Cu") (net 4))
 (segment (start 99.31 84.19) (end 99.425 84.19) (width 1) (layer "B.Cu") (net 4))
 (segment (start 91.5 87.25) (end 96.25 87.25) (width 1) (layer "B.Cu") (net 4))
 (segment (start 99.21 84.19) (end 99.425 84.19) (width 1) (layer "B.Cu") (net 4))
 (segment (start 96.25 87.25) (end 99.31 84.19) (width 1) (layer "B.Cu") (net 4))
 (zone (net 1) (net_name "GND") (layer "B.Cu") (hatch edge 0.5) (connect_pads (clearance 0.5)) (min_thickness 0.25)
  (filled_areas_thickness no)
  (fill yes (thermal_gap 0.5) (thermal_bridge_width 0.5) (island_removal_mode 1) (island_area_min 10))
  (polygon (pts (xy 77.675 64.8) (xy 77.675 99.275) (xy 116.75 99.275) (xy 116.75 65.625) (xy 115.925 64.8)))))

